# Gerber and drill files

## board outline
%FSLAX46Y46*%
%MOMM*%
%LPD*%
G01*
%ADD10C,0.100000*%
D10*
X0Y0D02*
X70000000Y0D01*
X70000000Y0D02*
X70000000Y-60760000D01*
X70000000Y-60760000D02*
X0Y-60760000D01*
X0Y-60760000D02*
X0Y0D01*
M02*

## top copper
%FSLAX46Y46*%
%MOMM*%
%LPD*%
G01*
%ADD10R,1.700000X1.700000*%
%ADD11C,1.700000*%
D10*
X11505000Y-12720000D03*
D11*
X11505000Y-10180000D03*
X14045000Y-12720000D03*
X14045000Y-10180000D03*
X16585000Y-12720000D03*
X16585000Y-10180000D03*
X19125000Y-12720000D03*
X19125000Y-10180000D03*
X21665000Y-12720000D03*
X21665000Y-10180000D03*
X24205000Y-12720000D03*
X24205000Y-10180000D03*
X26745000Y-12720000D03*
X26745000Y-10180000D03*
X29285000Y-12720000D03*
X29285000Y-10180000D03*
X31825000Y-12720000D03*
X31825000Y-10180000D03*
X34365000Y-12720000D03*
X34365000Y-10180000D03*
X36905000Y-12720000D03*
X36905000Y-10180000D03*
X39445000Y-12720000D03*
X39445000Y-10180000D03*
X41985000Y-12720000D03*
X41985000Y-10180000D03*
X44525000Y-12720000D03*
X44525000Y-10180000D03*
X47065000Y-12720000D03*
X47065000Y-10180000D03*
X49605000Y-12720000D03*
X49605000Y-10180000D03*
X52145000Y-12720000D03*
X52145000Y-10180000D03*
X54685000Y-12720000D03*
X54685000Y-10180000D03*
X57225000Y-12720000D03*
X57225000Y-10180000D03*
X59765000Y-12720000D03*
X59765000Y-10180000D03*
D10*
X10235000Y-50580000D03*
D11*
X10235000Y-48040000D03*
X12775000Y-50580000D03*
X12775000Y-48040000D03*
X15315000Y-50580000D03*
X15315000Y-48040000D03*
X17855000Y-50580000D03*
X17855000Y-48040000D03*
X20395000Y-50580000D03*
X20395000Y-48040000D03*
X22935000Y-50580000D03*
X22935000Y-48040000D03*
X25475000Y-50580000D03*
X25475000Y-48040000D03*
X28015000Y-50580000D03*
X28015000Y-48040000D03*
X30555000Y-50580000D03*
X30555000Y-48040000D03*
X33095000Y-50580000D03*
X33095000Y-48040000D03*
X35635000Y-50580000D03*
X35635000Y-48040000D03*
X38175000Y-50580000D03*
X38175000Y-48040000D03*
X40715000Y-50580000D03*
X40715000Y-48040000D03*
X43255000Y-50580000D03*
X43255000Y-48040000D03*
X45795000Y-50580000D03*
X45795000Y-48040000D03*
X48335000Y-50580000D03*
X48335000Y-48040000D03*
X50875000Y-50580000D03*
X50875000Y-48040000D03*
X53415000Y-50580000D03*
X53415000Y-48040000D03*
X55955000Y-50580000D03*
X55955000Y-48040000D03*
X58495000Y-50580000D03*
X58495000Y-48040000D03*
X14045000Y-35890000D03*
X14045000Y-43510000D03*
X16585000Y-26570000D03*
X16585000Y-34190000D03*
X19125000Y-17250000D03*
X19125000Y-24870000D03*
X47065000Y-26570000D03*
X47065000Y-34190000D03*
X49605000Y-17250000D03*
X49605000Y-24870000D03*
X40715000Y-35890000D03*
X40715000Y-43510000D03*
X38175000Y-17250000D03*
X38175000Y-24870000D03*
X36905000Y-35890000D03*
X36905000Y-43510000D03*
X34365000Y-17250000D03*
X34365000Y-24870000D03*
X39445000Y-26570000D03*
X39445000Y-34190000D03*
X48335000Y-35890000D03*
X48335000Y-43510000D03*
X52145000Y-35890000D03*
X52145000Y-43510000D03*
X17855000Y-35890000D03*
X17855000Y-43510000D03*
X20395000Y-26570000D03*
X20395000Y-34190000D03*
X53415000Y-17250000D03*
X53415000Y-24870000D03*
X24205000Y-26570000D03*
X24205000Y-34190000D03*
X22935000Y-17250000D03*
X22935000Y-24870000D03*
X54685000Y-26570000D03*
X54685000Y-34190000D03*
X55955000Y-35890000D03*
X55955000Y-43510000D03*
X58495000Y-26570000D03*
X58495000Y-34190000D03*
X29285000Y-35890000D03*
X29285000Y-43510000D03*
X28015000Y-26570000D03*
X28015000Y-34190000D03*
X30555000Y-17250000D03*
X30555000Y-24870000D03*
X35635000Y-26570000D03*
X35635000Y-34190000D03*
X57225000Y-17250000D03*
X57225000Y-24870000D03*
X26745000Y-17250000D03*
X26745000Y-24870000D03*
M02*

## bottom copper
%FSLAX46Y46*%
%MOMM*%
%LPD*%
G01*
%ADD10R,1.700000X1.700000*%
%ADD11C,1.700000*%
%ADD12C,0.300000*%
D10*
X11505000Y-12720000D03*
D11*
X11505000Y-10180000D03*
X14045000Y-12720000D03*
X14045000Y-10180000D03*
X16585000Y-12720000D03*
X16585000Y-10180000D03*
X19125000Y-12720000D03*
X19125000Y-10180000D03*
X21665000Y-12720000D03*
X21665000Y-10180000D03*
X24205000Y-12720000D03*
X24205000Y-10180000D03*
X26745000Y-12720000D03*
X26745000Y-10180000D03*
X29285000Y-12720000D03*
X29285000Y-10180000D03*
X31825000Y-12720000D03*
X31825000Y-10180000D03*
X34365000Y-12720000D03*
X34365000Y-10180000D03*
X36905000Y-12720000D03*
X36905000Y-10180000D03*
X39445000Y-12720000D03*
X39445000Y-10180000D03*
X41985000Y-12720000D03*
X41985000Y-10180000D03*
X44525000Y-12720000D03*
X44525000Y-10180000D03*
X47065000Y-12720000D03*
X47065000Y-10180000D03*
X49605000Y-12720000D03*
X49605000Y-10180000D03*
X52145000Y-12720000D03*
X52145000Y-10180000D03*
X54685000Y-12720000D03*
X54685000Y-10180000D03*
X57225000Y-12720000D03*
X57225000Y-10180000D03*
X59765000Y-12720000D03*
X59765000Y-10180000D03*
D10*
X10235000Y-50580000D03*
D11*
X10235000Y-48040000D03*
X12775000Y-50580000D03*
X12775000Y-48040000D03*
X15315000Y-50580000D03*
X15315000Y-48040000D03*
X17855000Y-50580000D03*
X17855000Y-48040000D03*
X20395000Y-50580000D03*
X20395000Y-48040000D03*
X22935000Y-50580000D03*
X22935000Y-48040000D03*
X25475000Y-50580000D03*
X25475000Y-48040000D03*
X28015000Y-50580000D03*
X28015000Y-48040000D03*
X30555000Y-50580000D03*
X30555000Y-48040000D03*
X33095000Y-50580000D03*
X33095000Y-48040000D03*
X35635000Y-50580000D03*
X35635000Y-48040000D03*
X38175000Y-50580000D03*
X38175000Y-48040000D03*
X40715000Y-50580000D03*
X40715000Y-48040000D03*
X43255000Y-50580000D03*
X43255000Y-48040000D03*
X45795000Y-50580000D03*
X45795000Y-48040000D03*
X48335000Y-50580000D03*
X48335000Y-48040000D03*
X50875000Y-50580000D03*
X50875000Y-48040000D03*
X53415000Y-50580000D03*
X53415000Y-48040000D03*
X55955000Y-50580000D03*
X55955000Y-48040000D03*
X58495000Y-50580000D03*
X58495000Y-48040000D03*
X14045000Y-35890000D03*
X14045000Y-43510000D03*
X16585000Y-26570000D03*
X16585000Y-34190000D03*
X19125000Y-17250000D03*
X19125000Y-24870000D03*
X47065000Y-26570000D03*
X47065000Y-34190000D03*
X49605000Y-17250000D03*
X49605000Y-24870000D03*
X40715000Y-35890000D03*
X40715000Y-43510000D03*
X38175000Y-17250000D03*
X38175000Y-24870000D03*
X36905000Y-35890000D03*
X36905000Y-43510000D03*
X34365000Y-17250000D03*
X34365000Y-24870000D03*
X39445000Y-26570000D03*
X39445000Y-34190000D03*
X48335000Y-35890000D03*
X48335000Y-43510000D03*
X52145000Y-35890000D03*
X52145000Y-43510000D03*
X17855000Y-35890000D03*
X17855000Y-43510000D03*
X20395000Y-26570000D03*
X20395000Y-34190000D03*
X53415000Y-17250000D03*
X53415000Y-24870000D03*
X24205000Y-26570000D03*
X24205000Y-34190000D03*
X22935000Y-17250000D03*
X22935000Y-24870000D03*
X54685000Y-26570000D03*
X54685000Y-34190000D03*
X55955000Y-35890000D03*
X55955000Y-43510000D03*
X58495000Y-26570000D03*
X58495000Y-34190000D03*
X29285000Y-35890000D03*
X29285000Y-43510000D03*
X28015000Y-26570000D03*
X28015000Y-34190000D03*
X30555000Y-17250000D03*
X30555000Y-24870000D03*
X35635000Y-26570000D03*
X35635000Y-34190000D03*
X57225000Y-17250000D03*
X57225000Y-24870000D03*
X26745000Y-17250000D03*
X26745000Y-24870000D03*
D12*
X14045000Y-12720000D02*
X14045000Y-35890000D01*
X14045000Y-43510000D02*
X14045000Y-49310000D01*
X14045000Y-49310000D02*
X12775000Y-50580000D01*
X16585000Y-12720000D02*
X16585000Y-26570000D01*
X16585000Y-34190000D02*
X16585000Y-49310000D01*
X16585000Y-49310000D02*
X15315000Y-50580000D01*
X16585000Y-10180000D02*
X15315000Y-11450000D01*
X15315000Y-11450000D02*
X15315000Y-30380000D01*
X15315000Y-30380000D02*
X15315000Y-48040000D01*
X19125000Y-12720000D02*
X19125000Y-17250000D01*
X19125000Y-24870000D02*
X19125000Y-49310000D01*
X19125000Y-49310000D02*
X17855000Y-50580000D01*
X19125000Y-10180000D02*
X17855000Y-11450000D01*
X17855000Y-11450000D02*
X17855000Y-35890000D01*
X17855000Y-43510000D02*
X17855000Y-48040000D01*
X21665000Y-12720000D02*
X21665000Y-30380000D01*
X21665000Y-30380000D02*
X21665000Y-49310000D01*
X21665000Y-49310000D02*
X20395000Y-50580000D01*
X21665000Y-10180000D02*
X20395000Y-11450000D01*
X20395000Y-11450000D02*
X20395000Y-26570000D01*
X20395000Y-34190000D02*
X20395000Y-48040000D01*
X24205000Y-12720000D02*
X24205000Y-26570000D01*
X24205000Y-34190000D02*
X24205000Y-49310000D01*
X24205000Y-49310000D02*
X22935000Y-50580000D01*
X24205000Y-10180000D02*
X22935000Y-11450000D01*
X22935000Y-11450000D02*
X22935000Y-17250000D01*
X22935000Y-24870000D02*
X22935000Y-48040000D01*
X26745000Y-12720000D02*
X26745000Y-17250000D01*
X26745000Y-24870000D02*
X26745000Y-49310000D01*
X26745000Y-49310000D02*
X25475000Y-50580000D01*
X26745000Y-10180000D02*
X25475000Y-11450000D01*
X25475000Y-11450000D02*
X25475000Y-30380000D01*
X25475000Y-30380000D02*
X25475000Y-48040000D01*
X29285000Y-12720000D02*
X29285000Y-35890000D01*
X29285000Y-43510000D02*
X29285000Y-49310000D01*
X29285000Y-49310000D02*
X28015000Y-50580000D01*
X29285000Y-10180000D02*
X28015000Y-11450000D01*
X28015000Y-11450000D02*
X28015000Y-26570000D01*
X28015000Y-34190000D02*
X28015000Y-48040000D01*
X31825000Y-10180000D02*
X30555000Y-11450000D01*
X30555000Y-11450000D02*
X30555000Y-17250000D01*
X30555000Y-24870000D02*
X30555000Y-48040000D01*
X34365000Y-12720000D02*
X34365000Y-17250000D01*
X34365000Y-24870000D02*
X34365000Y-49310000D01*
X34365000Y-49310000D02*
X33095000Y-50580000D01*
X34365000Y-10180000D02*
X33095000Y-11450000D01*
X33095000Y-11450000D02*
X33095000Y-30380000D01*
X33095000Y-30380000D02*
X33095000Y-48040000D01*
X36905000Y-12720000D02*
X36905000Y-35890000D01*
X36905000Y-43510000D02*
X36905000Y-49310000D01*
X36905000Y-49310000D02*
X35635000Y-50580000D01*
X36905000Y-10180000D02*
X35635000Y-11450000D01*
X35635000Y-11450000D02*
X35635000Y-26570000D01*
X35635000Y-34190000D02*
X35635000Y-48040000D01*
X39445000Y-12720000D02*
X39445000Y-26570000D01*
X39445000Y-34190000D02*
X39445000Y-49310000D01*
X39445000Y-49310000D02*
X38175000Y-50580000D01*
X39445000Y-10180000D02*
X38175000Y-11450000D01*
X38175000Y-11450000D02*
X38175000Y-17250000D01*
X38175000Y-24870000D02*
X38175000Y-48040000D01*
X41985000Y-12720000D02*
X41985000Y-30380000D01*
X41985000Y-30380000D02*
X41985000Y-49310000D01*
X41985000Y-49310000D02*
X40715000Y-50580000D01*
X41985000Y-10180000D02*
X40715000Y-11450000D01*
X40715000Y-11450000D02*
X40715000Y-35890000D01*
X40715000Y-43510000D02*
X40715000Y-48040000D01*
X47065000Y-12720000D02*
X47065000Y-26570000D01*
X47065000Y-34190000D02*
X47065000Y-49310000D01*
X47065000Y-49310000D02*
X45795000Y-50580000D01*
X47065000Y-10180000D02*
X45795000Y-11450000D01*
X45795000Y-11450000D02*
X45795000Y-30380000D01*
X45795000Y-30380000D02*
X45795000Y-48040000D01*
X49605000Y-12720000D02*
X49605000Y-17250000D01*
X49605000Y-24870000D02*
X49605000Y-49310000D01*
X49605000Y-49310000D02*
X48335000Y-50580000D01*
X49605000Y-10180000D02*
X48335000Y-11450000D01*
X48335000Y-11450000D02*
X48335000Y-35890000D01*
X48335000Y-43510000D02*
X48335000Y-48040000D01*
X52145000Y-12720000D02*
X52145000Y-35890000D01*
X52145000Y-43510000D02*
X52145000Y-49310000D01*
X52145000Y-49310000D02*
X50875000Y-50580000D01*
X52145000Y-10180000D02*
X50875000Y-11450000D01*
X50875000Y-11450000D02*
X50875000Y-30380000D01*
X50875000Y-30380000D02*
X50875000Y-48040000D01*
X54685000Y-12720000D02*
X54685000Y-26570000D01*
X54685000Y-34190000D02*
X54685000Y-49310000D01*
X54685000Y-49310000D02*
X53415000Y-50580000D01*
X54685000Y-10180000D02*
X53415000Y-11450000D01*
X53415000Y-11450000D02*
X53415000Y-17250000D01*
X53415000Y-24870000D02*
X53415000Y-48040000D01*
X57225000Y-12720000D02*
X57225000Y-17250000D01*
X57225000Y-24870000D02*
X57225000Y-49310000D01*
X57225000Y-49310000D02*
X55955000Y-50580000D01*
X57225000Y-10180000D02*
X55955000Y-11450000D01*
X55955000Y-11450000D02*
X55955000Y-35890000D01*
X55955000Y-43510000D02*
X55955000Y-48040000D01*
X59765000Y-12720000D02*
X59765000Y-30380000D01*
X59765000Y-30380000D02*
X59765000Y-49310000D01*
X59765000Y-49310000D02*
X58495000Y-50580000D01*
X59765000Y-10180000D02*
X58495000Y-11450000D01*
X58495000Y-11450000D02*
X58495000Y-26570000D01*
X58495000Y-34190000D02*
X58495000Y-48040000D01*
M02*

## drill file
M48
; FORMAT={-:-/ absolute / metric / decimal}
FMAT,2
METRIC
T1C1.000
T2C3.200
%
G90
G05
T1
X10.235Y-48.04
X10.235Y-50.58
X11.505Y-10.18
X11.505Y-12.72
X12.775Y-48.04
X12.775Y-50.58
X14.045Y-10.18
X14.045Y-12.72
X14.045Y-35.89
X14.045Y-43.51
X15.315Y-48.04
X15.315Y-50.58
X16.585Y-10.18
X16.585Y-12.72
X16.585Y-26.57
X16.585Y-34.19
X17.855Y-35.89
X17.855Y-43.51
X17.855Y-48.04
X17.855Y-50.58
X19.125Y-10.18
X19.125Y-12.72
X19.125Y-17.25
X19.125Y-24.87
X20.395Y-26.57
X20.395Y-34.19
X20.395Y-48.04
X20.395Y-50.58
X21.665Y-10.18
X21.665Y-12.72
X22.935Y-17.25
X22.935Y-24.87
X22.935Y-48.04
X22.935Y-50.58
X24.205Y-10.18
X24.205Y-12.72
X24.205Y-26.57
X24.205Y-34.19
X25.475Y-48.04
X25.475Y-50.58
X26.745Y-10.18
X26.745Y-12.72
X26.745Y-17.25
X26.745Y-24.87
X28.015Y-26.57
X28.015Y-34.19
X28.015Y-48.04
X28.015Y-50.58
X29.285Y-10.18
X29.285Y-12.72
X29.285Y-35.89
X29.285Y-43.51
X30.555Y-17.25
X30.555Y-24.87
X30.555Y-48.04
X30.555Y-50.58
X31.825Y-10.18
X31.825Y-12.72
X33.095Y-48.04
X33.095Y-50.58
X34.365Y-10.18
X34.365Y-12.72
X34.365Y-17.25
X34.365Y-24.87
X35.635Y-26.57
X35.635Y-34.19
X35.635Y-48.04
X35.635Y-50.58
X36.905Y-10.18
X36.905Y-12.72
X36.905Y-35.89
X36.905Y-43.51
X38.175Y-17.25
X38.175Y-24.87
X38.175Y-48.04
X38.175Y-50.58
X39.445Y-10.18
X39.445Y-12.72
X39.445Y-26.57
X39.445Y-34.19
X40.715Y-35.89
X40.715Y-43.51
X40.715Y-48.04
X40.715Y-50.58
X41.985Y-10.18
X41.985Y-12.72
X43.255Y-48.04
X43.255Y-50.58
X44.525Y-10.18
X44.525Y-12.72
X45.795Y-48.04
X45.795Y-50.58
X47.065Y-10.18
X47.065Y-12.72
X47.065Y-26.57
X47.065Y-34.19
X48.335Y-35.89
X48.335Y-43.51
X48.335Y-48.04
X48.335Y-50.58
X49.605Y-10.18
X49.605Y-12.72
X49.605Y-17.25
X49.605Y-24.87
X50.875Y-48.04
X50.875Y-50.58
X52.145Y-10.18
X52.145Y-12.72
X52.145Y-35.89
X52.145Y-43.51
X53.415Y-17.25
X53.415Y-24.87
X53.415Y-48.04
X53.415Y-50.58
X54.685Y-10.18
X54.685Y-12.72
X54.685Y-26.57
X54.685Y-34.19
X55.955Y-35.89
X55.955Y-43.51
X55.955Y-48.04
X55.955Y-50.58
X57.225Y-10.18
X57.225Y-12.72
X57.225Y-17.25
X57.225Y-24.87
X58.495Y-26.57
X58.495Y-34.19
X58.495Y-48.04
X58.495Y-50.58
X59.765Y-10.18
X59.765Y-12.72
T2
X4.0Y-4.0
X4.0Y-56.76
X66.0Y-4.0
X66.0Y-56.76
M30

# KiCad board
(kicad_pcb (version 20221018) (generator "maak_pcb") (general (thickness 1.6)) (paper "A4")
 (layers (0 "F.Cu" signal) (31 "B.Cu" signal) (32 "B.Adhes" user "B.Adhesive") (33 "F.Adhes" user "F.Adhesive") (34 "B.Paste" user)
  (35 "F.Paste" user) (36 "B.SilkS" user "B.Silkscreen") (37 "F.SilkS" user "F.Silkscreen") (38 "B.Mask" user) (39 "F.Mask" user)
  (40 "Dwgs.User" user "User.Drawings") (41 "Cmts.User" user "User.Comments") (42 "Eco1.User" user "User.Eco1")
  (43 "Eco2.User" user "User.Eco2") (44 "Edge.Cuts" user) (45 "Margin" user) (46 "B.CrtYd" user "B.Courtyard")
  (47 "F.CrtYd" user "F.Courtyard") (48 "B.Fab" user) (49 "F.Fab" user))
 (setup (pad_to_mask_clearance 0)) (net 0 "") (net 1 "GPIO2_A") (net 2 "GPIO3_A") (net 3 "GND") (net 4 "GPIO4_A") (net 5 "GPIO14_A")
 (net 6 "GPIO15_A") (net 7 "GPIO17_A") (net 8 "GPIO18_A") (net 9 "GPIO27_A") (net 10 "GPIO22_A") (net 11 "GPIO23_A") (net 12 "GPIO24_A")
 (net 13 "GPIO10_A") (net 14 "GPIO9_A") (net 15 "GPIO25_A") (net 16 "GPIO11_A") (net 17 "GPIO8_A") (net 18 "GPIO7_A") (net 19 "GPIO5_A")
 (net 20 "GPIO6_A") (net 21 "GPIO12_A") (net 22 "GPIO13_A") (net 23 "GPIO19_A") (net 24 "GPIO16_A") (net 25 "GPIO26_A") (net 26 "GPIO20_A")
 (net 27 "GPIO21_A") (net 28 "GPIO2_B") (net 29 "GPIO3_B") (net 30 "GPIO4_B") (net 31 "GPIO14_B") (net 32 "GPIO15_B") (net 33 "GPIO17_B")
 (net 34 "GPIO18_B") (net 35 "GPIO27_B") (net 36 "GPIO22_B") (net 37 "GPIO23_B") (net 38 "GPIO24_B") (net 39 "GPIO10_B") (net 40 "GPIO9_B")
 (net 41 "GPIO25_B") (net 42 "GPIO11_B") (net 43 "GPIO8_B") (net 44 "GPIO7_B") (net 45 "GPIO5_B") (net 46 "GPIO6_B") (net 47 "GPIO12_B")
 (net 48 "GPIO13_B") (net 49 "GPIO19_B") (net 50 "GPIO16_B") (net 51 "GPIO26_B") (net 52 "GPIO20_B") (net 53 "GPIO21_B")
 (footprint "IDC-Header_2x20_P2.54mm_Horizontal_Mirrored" (layer "F.Cu") (at 11.505 12.72)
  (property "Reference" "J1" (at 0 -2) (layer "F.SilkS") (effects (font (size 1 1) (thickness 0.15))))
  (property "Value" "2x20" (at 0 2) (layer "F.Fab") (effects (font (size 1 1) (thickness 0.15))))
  (pad "1" thru_hole rect (at 0 0) (size 1.7 1.7) (drill 1) (layers "B.Cu" "B.Mask"))
  (pad "2" thru_hole circle (at 0 -2.54) (size 1.7 1.7) (drill 1) (layers "B.Cu" "B.Mask"))
  (pad "3" thru_hole circle (at 2.54 0) (size 1.7 1.7) (drill 1) (layers "B.Cu" "B.Mask") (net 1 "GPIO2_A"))
  (pad "4" thru_hole circle (at 2.54 -2.54) (size 1.7 1.7) (drill 1) (layers "B.Cu" "B.Mask"))
  (pad "5" thru_hole circle (at 5.08 0) (size 1.7 1.7) (drill 1) (layers "B.Cu" "B.Mask") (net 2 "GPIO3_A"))
  (pad "6" thru_hole circle (at 5.08 -2.54) (size 1.7 1.7) (drill 1) (layers "B.Cu" "B.Mask") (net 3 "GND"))
  (pad "7" thru_hole circle (at 7.62 0) (size 1.7 1.7) (drill 1) (layers "B.Cu" "B.Mask") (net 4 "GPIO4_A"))
  (pad "8" thru_hole circle (at 7.62 -2.54) (size 1.7 1.7) (drill 1) (layers "B.Cu" "B.Mask") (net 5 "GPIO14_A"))
  (pad "9" thru_hole circle (at 10.16 0) (size 1.7 1.7) (drill 1) (layers "B.Cu" "B.Mask") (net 3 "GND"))
  (pad "10" thru_hole circle (at 10.16 -2.54) (size 1.7 1.7) (drill 1) (layers "B.Cu" "B.Mask") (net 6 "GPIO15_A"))
  (pad "11" thru_hole circle (at 12.7 0) (size 1.7 1.7) (drill 1) (layers "B.Cu" "B.Mask") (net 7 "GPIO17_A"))
  (pad "12" thru_hole circle (at 12.7 -2.54) (size 1.7 1.7) (drill 1) (layers "B.Cu" "B.Mask") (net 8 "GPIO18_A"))
  (pad "13" thru_hole circle (at 15.24 0) (size 1.7 1.7) (drill 1) (layers "B.Cu" "B.Mask") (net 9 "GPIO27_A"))
  (pad "14" thru_hole circle (at 15.24 -2.54) (size 1.7 1.7) (drill 1) (layers "B.Cu" "B.Mask") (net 3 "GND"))
  (pad "15" thru_hole circle (at 17.78 0) (size 1.7 1.7) (drill 1) (layers "B.Cu" "B.Mask") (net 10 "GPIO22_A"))
  (pad "16" thru_hole circle (at 17.78 -2.54) (size 1.7 1.7) (drill 1) (layers "B.Cu" "B.Mask") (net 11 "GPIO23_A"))
  (pad "17" thru_hole circle (at 20.32 0) (size 1.7 1.7) (drill 1) (layers "B.Cu" "B.Mask"))
  (pad "18" thru_hole circle (at 20.32 -2.54) (size 1.7 1.7) (drill 1) (layers "B.Cu" "B.Mask") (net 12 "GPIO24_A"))
  (pad "19" thru_hole circle (at 22.86 0) (size 1.7 1.7) (drill 1) (layers "B.Cu" "B.Mask") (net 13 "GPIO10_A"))
  (pad "20" thru_hole circle (at 22.86 -2.54) (size 1.7 1.7) (drill 1) (layers "B.Cu" "B.Mask") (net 3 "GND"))
  (pad "21" thru_hole circle (at 25.4 0) (size 1.7 1.7) (drill 1) (layers "B.Cu" "B.Mask") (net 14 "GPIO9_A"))
  (pad "22" thru_hole circle (at 25.4 -2.54) (size 1.7 1.7) (drill 1) (layers "B.Cu" "B.Mask") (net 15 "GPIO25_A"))
  (pad "23" thru_hole circle (at 27.94 0) (size 1.7 1.7) (drill 1) (layers "B.Cu" "B.Mask") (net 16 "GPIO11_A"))
  (pad "24" thru_hole circle (at 27.94 -2.54) (size 1.7 1.7) (drill 1) (layers "B.Cu" "B.Mask") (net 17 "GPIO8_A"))
  (pad "25" thru_hole circle (at 30.48 0) (size 1.7 1.7) (drill 1) (layers "B.Cu" "B.Mask") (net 3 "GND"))
  (pad "26" thru_hole circle (at 30.48 -2.54) (size 1.7 1.7) (drill 1) (layers "B.Cu" "B.Mask") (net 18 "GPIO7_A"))
  (pad "27" thru_hole circle (at 33.02 0) (size 1.7 1.7) (drill 1) (layers "B.Cu" "B.Mask"))
  (pad "28" thru_hole circle (at 33.02 -2.54) (size 1.7 1.7) (drill 1) (layers "B.Cu" "B.Mask"))
  (pad "29" thru_hole circle (at 35.56 0) (size 1.7 1.7) (drill 1) (layers "B.Cu" "B.Mask") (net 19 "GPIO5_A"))
  (pad "30" thru_hole circle (at 35.56 -2.54) (size 1.7 1.7) (drill 1) (layers "B.Cu" "B.Mask") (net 3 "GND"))
  (pad "31" thru_hole circle (at 38.1 0) (size 1.7 1.7) (drill 1) (layers "B.Cu" "B.Mask") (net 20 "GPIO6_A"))
  (pad "32" thru_hole circle (at 38.1 -2.54) (size 1.7 1.7) (drill 1) (layers "B.Cu" "B.Mask") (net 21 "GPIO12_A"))
  (pad "33" thru_hole circle (at 40.64 0) (size 1.7 1.7) (drill 1) (layers "B.Cu" "B.Mask") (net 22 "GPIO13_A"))
  (pad "34" thru_hole circle (at 40.64 -2.54) (size 1.7 1.7) (drill 1) (layers "B.Cu" "B.Mask") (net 3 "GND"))
  (pad "35" thru_hole circle (at 43.18 0) (size 1.7 1.7) (drill 1) (layers "B.Cu" "B.Mask") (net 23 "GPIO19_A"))
  (pad "36" thru_hole circle (at 43.18 -2.54) (size 1.7 1.7) (drill 1) (layers "B.Cu" "B.Mask") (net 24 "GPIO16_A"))
  (pad "37" thru_hole circle (at 45.72 0) (size 1.7 1.7) (drill 1) (layers "B.Cu" "B.Mask") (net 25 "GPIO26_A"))
  (pad "38" thru_hole circle (at 45.72 -2.54) (size 1.7 1.7) (drill 1) (layers "B.Cu" "B.Mask") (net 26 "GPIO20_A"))
  (pad "39" thru_hole circle (at 48.26 0) (size 1.7 1.7) (drill 1) (layers "B.Cu" "B.Mask") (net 3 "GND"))
  (pad "40" thru_hole circle (at 48.26 -2.54) (size 1.7 1.7) (drill 1) (layers "B.Cu" "B.Mask") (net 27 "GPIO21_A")))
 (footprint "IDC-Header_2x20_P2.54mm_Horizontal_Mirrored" (layer "F.Cu") (at 10.235 50.58)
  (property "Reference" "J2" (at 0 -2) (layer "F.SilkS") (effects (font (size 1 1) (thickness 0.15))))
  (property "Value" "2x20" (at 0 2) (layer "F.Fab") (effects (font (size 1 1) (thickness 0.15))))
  (pad "1" thru_hole rect (at 0 0) (size 1.7 1.7) (drill 1) (layers "B.Cu" "B.Mask"))
  (pad "2" thru_hole circle (at 0 -2.54) (size 1.7 1.7) (drill 1) (layers "B.Cu" "B.Mask"))
  (pad "3" thru_hole circle (at 2.54 0) (size 1.7 1.7) (drill 1) (layers "B.Cu" "B.Mask") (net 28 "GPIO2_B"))
  (pad "4" thru_hole circle (at 2.54 -2.54) (size 1.7 1.7) (drill 1) (layers "B.Cu" "B.Mask"))
  (pad "5" thru_hole circle (at 5.08 0) (size 1.7 1.7) (drill 1) (layers "B.Cu" "B.Mask") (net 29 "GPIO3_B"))
  (pad "6" thru_hole circle (at 5.08 -2.54) (size 1.7 1.7) (drill 1) (layers "B.Cu" "B.Mask") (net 3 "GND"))
  (pad "7" thru_hole circle (at 7.62 0) (size 1.7 1.7) (drill 1) (layers "B.Cu" "B.Mask") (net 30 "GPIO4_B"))
  (pad "8" thru_hole circle (at 7.62 -2.54) (size 1.7 1.7) (drill 1) (layers "B.Cu" "B.Mask") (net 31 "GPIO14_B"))
  (pad "9" thru_hole circle (at 10.16 0) (size 1.7 1.7) (drill 1) (layers "B.Cu" "B.Mask") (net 3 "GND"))
  (pad "10" thru_hole circle (at 10.16 -2.54) (size 1.7 1.7) (drill 1) (layers "B.Cu" "B.Mask") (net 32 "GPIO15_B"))
  (pad "11" thru_hole circle (at 12.7 0) (size 1.7 1.7) (drill 1) (layers "B.Cu" "B.Mask") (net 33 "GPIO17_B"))
  (pad "12" thru_hole circle (at 12.7 -2.54) (size 1.7 1.7) (drill 1) (layers "B.Cu" "B.Mask") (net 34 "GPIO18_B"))
  (pad "13" thru_hole circle (at 15.24 0) (size 1.7 1.7) (drill 1) (layers "B.Cu" "B.Mask") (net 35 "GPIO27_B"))
  (pad "14" thru_hole circle (at 15.24 -2.54) (size 1.7 1.7) (drill 1) (layers "B.Cu" "B.Mask") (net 3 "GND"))
  (pad "15" thru_hole circle (at 17.78 0) (size 1.7 1.7) (drill 1) (layers "B.Cu" "B.Mask") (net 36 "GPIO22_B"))
  (pad "16" thru_hole circle (at 17.78 -2.54) (size 1.7 1.7) (drill 1) (layers "B.Cu" "B.Mask") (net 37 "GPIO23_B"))
  (pad "17" thru_hole circle (at 20.32 0) (size 1.7 1.7) (drill 1) (layers "B.Cu" "B.Mask"))
  (pad "18" thru_hole circle (at 20.32 -2.54) (size 1.7 1.7) (drill 1) (layers "B.Cu" "B.Mask") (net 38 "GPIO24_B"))
  (pad "19" thru_hole circle (at 22.86 0) (size 1.7 1.7) (drill 1) (layers "B.Cu" "B.Mask") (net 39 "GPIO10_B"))
  (pad "20" thru_hole circle (at 22.86 -2.54) (size 1.7 1.7) (drill 1) (layers "B.Cu" "B.Mask") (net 3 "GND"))
  (pad "21" thru_hole circle (at 25.4 0) (size 1.7 1.7) (drill 1) (layers "B.Cu" "B.Mask") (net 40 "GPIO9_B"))
  (pad "22" thru_hole circle (at 25.4 -2.54) (size 1.7 1.7) (drill 1) (layers "B.Cu" "B.Mask") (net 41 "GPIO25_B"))
  (pad "23" thru_hole circle (at 27.94 0) (size 1.7 1.7) (drill 1) (layers "B.Cu" "B.Mask") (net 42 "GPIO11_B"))
  (pad "24" thru_hole circle (at 27.94 -2.54) (size 1.7 1.7) (drill 1) (layers "B.Cu" "B.Mask") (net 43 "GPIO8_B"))
  (pad "25" thru_hole circle (at 30.48 0) (size 1.7 1.7) (drill 1) (layers "B.Cu" "B.Mask") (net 3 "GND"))
  (pad "26" thru_hole circle (at 30.48 -2.54) (size 1.7 1.7) (drill 1) (layers "B.Cu" "B.Mask") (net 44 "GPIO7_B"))
  (pad "27" thru_hole circle (at 33.02 0) (size 1.7 1.7) (drill 1) (layers "B.Cu" "B.Mask"))
  (pad "28" thru_hole circle (at 33.02 -2.54) (size 1.7 1.7) (drill 1) (layers "B.Cu" "B.Mask"))
  (pad "29" thru_hole circle (at 35.56 0) (size 1.7 1.7) (drill 1) (layers "B.Cu" "B.Mask") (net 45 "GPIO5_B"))
  (pad "30" thru_hole circle (at 35.56 -2.54) (size 1.7 1.7) (drill 1) (layers "B.Cu" "B.Mask") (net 3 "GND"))
  (pad "31" thru_hole circle (at 38.1 0) (size 1.7 1.7) (drill 1) (layers "B.Cu" "B.Mask") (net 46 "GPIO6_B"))
  (pad "32" thru_hole circle (at 38.1 -2.54) (size 1.7 1.7) (drill 1) (layers "B.Cu" "B.Mask") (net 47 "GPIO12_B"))
  (pad "33" thru_hole circle (at 40.64 0) (size 1.7 1.7) (drill 1) (layers "B.Cu" "B.Mask") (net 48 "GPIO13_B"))
  (pad "34" thru_hole circle (at 40.64 -2.54) (size 1.7 1.7) (drill 1) (layers "B.Cu" "B.Mask") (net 3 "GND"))
  (pad "35" thru_hole circle (at 43.18 0) (size 1.7 1.7) (drill 1) (layers "B.Cu" "B.Mask") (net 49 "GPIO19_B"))
  (pad "36" thru_hole circle (at 43.18 -2.54) (size 1.7 1.7) (drill 1) (layers "B.Cu" "B.Mask") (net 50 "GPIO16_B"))
  (pad "37" thru_hole circle (at 45.72 0) (size 1.7 1.7) (drill 1) (layers "B.Cu" "B.Mask") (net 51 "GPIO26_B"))
  (pad "38" thru_hole circle (at 45.72 -2.54) (size 1.7 1.7) (drill 1) (layers "B.Cu" "B.Mask") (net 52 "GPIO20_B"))
  (pad "39" thru_hole circle (at 48.26 0) (size 1.7 1.7) (drill 1) (layers "B.Cu" "B.Mask") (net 3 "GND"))
  (pad "40" thru_hole circle (at 48.26 -2.54) (size 1.7 1.7) (drill 1) (layers "B.Cu" "B.Mask") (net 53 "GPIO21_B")))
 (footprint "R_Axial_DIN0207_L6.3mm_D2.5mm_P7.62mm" (layer "F.Cu") (at 14.045 35.89)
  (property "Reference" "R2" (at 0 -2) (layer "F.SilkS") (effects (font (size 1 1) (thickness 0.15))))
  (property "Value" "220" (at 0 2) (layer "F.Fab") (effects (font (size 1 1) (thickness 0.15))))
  (pad "1" thru_hole circle (at 0 0) (size 1.7 1.7) (drill 1) (layers "B.Cu" "B.Mask") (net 1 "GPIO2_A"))
  (pad "2" thru_hole circle (at 0 7.62) (size 1.7 1.7) (drill 1) (layers "B.Cu" "B.Mask") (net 28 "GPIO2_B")))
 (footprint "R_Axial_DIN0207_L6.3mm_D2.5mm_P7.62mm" (layer "F.Cu") (at 16.585 26.57)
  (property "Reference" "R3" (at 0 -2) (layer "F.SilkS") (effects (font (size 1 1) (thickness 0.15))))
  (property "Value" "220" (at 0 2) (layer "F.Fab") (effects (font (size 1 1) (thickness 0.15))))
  (pad "1" thru_hole circle (at 0 0) (size 1.7 1.7) (drill 1) (layers "B.Cu" "B.Mask") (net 2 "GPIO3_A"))
  (pad "2" thru_hole circle (at 0 7.62) (size 1.7 1.7) (drill 1) (layers "B.Cu" "B.Mask") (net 29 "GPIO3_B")))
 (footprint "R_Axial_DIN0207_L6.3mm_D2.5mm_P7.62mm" (layer "F.Cu") (at 19.125 17.25)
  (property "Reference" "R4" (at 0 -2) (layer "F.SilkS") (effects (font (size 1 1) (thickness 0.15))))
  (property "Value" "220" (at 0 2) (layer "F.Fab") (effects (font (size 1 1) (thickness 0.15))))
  (pad "1" thru_hole circle (at 0 0) (size 1.7 1.7) (drill 1) (layers "B.Cu" "B.Mask") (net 4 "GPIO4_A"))
  (pad "2" thru_hole circle (at 0 7.62) (size 1.7 1.7) (drill 1) (layers "B.Cu" "B.Mask") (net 30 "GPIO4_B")))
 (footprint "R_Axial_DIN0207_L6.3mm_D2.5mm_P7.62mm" (layer "F.Cu") (at 47.065 26.57)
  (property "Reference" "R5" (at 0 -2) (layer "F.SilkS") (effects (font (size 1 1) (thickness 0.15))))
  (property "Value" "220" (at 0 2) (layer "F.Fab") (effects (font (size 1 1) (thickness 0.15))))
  (pad "1" thru_hole circle (at 0 0) (size 1.7 1.7) (drill 1) (layers "B.Cu" "B.Mask") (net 19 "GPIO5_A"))
  (pad "2" thru_hole circle (at 0 7.62) (size 1.7 1.7) (drill 1) (layers "B.Cu" "B.Mask") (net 45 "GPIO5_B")))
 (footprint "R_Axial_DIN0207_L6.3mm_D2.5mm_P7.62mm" (layer "F.Cu") (at 49.605 17.25)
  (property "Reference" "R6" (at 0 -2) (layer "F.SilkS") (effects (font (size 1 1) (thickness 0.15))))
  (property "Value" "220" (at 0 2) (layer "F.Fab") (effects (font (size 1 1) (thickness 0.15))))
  (pad "1" thru_hole circle (at 0 0) (size 1.7 1.7) (drill 1) (layers "B.Cu" "B.Mask") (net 20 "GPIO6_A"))
  (pad "2" thru_hole circle (at 0 7.62) (size 1.7 1.7) (drill 1) (layers "B.Cu" "B.Mask") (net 46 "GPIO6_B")))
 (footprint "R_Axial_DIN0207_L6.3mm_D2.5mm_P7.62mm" (layer "F.Cu") (at 40.715 35.89)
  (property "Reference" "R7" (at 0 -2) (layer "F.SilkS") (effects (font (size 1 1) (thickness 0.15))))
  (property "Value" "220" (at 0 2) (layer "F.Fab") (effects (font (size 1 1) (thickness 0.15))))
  (pad "1" thru_hole circle (at 0 0) (size 1.7 1.7) (drill 1) (layers "B.Cu" "B.Mask") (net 18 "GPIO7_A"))
  (pad "2" thru_hole circle (at 0 7.62) (size 1.7 1.7) (drill 1) (layers "B.Cu" "B.Mask") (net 44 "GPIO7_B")))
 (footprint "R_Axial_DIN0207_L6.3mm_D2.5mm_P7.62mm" (layer "F.Cu") (at 38.175 17.25)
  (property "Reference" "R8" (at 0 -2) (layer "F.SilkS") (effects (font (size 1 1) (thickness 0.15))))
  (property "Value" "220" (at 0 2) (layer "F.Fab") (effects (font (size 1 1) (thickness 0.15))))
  (pad "1" thru_hole circle (at 0 0) (size 1.7 1.7) (drill 1) (layers "B.Cu" "B.Mask") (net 17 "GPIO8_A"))
  (pad "2" thru_hole circle (at 0 7.62) (size 1.7 1.7) (drill 1) (layers "B.Cu" "B.Mask") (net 43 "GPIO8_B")))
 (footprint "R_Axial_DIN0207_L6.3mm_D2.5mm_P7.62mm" (layer "F.Cu") (at 36.905 35.89)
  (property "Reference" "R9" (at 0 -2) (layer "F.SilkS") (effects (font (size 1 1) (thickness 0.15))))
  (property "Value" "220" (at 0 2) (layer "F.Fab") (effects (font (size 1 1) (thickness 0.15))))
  (pad "1" thru_hole circle (at 0 0) (size 1.7 1.7) (drill 1) (layers "B.Cu" "B.Mask") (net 14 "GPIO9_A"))
  (pad "2" thru_hole circle (at 0 7.62) (size 1.7 1.7) (drill 1) (layers "B.Cu" "B.Mask") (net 40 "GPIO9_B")))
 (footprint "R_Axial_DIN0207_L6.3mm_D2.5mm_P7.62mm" (layer "F.Cu") (at 34.365 17.25)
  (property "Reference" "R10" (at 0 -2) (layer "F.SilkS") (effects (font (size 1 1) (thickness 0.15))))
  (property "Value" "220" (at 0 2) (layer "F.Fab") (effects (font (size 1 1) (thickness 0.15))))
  (pad "1" thru_hole circle (at 0 0) (size 1.7 1.7) (drill 1) (layers "B.Cu" "B.Mask") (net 13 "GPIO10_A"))
  (pad "2" thru_hole circle (at 0 7.62) (size 1.7 1.7) (drill 1) (layers "B.Cu" "B.Mask") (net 39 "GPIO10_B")))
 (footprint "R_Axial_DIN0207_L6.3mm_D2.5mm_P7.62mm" (layer "F.Cu") (at 39.445 26.57)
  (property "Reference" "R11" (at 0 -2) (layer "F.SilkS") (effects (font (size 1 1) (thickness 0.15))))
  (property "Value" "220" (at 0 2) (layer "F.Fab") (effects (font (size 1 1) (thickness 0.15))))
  (pad "1" thru_hole circle (at 0 0) (size 1.7 1.7) (drill 1) (layers "B.Cu" "B.Mask") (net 16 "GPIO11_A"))
  (pad "2" thru_hole circle (at 0 7.62) (size 1.7 1.7) (drill 1) (layers "B.Cu" "B.Mask") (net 42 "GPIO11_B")))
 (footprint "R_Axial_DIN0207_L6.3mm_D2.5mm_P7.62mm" (layer "F.Cu") (at 48.335 35.89)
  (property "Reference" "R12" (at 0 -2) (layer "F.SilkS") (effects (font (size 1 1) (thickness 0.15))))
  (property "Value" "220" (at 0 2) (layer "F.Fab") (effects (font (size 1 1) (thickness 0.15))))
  (pad "1" thru_hole circle (at 0 0) (size 1.7 1.7) (drill 1) (layers "B.Cu" "B.Mask") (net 21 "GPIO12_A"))
  (pad "2" thru_hole circle (at 0 7.62) (size 1.7 1.7) (drill 1) (layers "B.Cu" "B.Mask") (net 47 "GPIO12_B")))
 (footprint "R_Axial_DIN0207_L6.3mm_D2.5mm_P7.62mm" (layer "F.Cu") (at 52.145 35.89)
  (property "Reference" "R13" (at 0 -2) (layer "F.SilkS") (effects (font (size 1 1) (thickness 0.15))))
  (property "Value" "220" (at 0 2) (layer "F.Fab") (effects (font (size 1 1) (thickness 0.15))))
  (pad "1" thru_hole circle (at 0 0) (size 1.7 1.7) (drill 1) (layers "B.Cu" "B.Mask") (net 22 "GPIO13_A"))
  (pad "2" thru_hole circle (at 0 7.62) (size 1.7 1.7) (drill 1) (layers "B.Cu" "B.Mask") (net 48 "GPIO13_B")))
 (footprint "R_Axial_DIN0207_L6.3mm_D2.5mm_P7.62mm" (layer "F.Cu") (at 17.855 35.89)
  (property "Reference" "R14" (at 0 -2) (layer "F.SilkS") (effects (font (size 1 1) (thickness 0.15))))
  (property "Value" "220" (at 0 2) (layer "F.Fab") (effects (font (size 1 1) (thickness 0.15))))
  (pad "1" thru_hole circle (at 0 0) (size 1.7 1.7) (drill 1) (layers "B.Cu" "B.Mask") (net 5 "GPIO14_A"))
  (pad "2" thru_hole circle (at 0 7.62) (size 1.7 1.7) (drill 1) (layers "B.Cu" "B.Mask") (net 31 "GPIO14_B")))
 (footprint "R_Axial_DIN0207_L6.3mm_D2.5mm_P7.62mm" (layer "F.Cu") (at 20.395 26.57)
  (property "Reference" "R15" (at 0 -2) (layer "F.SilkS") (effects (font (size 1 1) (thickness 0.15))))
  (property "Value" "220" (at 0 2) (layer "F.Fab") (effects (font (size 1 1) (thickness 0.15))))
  (pad "1" thru_hole circle (at 0 0) (size 1.7 1.7) (drill 1) (layers "B.Cu" "B.Mask") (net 6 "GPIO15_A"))
  (pad "2" thru_hole circle (at 0 7.62) (size 1.7 1.7) (drill 1) (layers "B.Cu" "B.Mask") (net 32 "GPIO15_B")))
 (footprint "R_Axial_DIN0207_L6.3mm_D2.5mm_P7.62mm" (layer "F.Cu") (at 53.415 17.25)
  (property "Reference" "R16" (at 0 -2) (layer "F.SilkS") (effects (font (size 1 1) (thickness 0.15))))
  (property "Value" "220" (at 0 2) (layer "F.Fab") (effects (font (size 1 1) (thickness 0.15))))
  (pad "1" thru_hole circle (at 0 0) (size 1.7 1.7) (drill 1) (layers "B.Cu" "B.Mask") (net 24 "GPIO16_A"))
  (pad "2" thru_hole circle (at 0 7.62) (size 1.7 1.7) (drill 1) (layers "B.Cu" "B.Mask") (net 50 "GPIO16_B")))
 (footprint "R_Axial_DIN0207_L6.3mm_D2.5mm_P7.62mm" (layer "F.Cu") (at 24.205 26.57)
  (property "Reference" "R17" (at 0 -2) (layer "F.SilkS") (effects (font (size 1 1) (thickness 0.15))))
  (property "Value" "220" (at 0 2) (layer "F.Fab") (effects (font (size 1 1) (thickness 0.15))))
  (pad "1" thru_hole circle (at 0 0) (size 1.7 1.7) (drill 1) (layers "B.Cu" "B.Mask") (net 7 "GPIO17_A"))
  (pad "2" thru_hole circle (at 0 7.62) (size 1.7 1.7) (drill 1) (layers "B.Cu" "B.Mask") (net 33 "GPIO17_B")))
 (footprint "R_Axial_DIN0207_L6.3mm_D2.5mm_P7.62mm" (layer "F.Cu") (at 22.935 17.25)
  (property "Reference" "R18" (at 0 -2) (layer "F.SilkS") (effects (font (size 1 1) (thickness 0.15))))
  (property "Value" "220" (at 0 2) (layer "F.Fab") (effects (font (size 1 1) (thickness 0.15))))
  (pad "1" thru_hole circle (at 0 0) (size 1.7 1.7) (drill 1) (layers "B.Cu" "B.Mask") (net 8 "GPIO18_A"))
  (pad "2" thru_hole circle (at 0 7.62) (size 1.7 1.7) (drill 1) (layers "B.Cu" "B.Mask") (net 34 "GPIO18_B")))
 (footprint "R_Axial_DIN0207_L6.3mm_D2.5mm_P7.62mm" (layer "F.Cu") (at 54.685 26.57)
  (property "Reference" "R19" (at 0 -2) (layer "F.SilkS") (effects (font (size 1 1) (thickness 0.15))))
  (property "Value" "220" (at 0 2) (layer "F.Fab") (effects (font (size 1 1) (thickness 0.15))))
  (pad "1" thru_hole circle (at 0 0) (size 1.7 1.7) (drill 1) (layers "B.Cu" "B.Mask") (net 23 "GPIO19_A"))
  (pad "2" thru_hole circle (at 0 7.62) (size 1.7 1.7) (drill 1) (layers "B.Cu" "B.Mask") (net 49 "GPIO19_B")))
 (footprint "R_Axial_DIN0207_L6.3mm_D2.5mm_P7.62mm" (layer "F.Cu") (at 55.955 35.89)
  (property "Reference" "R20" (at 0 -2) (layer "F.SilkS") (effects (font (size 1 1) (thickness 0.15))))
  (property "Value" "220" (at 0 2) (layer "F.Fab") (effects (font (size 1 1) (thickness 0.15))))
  (pad "1" thru_hole circle (at 0 0) (size 1.7 1.7) (drill 1) (layers "B.Cu" "B.Mask") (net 26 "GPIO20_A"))
  (pad "2" thru_hole circle (at 0 7.62) (size 1.7 1.7) (drill 1) (layers "B.Cu" "B.Mask") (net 52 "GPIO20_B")))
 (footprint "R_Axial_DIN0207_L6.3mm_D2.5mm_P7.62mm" (layer "F.Cu") (at 58.495 26.57)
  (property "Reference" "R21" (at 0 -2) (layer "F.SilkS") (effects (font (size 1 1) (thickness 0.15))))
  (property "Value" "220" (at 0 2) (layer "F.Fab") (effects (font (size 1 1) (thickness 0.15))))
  (pad "1" thru_hole circle (at 0 0) (size 1.7 1.7) (drill 1) (layers "B.Cu" "B.Mask") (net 27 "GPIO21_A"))
  (pad "2" thru_hole circle (at 0 7.62) (size 1.7 1.7) (drill 1) (layers "B.Cu" "B.Mask") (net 53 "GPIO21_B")))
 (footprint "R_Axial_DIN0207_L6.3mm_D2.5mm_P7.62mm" (layer "F.Cu") (at 29.285 35.89)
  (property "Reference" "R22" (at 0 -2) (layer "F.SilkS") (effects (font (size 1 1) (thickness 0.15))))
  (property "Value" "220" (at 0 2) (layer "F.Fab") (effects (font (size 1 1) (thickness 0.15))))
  (pad "1" thru_hole circle (at 0 0) (size 1.7 1.7) (drill 1) (layers "B.Cu" "B.Mask") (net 10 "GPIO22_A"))
  (pad "2" thru_hole circle (at 0 7.62) (size 1.7 1.7) (drill 1) (layers "B.Cu" "B.Mask") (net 36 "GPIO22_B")))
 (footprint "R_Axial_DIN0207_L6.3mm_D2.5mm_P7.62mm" (layer "F.Cu") (at 28.015 26.57)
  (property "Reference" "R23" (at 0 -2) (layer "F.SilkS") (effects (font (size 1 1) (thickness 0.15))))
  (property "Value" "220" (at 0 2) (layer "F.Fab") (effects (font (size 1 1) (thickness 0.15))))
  (pad "1" thru_hole circle (at 0 0) (size 1.7 1.7) (drill 1) (layers "B.Cu" "B.Mask") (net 11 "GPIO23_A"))
  (pad "2" thru_hole circle (at 0 7.62) (size 1.7 1.7) (drill 1) (layers "B.Cu" "B.Mask") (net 37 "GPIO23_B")))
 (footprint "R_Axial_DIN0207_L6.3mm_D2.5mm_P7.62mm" (layer "F.Cu") (at 30.555 17.25)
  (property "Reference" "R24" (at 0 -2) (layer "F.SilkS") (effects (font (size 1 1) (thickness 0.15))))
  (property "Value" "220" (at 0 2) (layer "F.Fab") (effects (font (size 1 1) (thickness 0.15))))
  (pad "1" thru_hole circle (at 0 0) (size 1.7 1.7) (drill 1) (layers "B.Cu" "B.Mask") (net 12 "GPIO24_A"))
  (pad "2" thru_hole circle (at 0 7.62) (size 1.7 1.7) (drill 1) (layers "B.Cu" "B.Mask") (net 38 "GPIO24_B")))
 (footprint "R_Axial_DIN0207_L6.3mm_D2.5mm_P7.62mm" (layer "F.Cu") (at 35.635 26.57)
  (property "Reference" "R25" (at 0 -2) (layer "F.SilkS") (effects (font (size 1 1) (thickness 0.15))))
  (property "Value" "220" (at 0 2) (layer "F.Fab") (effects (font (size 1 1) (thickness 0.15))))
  (pad "1" thru_hole circle (at 0 0) (size 1.7 1.7) (drill 1) (layers "B.Cu" "B.Mask") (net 15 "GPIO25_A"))
  (pad "2" thru_hole circle (at 0 7.62) (size 1.7 1.7) (drill 1) (layers "B.Cu" "B.Mask") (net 41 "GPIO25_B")))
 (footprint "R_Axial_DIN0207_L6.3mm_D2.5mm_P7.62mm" (layer "F.Cu") (at 57.225 17.25)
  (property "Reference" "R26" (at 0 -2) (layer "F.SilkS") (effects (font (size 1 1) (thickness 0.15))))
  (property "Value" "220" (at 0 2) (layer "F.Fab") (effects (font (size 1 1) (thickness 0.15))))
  (pad "1" thru_hole circle (at 0 0) (size 1.7 1.7) (drill 1) (layers "B.Cu" "B.Mask") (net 25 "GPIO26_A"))
  (pad "2" thru_hole circle (at 0 7.62) (size 1.7 1.7) (drill 1) (layers "B.Cu" "B.Mask") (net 51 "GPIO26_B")))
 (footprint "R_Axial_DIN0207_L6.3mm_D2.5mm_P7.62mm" (layer "F.Cu") (at 26.745 17.25)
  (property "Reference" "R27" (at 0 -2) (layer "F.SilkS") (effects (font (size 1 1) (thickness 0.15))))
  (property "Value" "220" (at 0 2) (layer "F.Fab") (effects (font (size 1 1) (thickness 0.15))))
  (pad "1" thru_hole circle (at 0 0) (size 1.7 1.7) (drill 1) (layers "B.Cu" "B.Mask") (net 9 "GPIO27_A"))
  (pad "2" thru_hole circle (at 0 7.62) (size 1.7 1.7) (drill 1) (layers "B.Cu" "B.Mask") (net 35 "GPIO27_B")))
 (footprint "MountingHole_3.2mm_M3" (layer "F.Cu") (at 4 4)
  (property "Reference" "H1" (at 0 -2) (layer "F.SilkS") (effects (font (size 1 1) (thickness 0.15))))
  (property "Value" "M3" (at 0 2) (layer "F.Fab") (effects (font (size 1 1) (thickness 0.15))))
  (pad "" np_thru_hole circle (at 0 0) (size 3.2 3.2) (drill 3.2) (layers "*.Cu" "*.Mask")))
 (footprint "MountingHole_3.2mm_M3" (layer "F.Cu") (at 66 4)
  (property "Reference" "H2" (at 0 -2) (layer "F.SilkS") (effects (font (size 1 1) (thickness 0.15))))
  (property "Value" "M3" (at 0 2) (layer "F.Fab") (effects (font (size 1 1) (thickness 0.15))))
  (pad "" np_thru_hole circle (at 0 0) (size 3.2 3.2) (drill 3.2) (layers "*.Cu" "*.Mask")))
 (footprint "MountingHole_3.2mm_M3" (layer "F.Cu") (at 4 56.76)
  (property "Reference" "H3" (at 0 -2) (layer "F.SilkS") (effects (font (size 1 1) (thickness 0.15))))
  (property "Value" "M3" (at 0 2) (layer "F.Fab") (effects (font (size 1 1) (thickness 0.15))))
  (pad "" np_thru_hole circle (at 0 0) (size 3.2 3.2) (drill 3.2) (layers "*.Cu" "*.Mask")))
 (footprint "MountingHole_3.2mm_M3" (layer "F.Cu") (at 66 56.76)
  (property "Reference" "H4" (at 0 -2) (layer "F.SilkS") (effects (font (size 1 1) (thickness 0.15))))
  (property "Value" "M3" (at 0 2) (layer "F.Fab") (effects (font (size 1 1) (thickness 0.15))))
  (pad "" np_thru_hole circle (at 0 0) (size 3.2 3.2) (drill 3.2) (layers "*.Cu" "*.Mask")))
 (segment (start 14.045 12.72) (end 14.045 35.89) (width 0.3) (layer "B.Cu") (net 1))
 (segment (start 14.045 43.51) (end 14.045 49.31) (width 0.3) (layer "B.Cu") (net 28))
 (segment (start 14.045 49.31) (end 12.775 50.58) (width 0.3) (layer "B.Cu") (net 28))
 (segment (start 16.585 12.72) (end 16.585 26.57) (width 0.3) (layer "B.Cu") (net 2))
 (segment (start 16.585 34.19) (end 16.585 49.31) (width 0.3) (layer "B.Cu") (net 29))
 (segment (start 16.585 49.31) (end 15.315 50.58) (width 0.3) (layer "B.Cu") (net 29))
 (segment (start 16.585 10.18) (end 15.315 11.45) (width 0.3) (layer "B.Cu") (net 3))
 (segment (start 15.315 11.45) (end 15.315 30.38) (width 0.3) (layer "B.Cu") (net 3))
 (segment (start 15.315 30.38) (end 15.315 48.04) (width 0.3) (layer "B.Cu") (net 3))
 (segment (start 19.125 12.72) (end 19.125 17.25) (width 0.3) (layer "B.Cu") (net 4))
 (segment (start 19.125 24.87) (end 19.125 49.31) (width 0.3) (layer "B.Cu") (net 30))
 (segment (start 19.125 49.31) (end 17.855 50.58) (width 0.3) (layer "B.Cu") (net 30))
 (segment (start 19.125 10.18) (end 17.855 11.45) (width 0.3) (layer "B.Cu") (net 5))
 (segment (start 17.855 11.45) (end 17.855 35.89) (width 0.3) (layer "B.Cu") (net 5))
 (segment (start 17.855 43.51) (end 17.855 48.04) (width 0.3) (layer "B.Cu") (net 31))
 (segment (start 21.665 12.72) (end 21.665 30.38) (width 0.3) (layer "B.Cu") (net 3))
 (segment (start 21.665 30.38) (end 21.665 49.31) (width 0.3) (layer "B.Cu") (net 3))
 (segment (start 21.665 49.31) (end 20.395 50.58) (width 0.3) (layer "B.Cu") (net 3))
 (segment (start 21.665 10.18) (end 20.395 11.45) (width 0.3) (layer "B.Cu") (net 6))
 (segment (start 20.395 11.45) (end 20.395 26.57) (width 0.3) (layer "B.Cu") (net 6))
 (segment (start 20.395 34.19) (end 20.395 48.04) (width 0.3) (layer "B.Cu") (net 32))
 (segment (start 24.205 12.72) (end 24.205 26.57) (width 0.3) (layer "B.Cu") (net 7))
 (segment (start 24.205 34.19) (end 24.205 49.31) (width 0.3) (layer "B.Cu") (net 33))
 (segment (start 24.205 49.31) (end 22.935 50.58) (width 0.3) (layer "B.Cu") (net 33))
 (segment (start 24.205 10.18) (end 22.935 11.45) (width 0.3) (layer "B.Cu") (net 8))
 (segment (start 22.935 11.45) (end 22.935 17.25) (width 0.3) (layer "B.Cu") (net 8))
 (segment (start 22.935 24.87) (end 22.935 48.04) (width 0.3) (layer "B.Cu") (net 34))
 (segment (start 26.745 12.72) (end 26.745 17.25) (width 0.3) (layer "B.Cu") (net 9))
 (segment (start 26.745 24.87) (end 26.745 49.31) (width 0.3) (layer "B.Cu") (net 35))
 (segment (start 26.745 49.31) (end 25.475 50.58) (width 0.3) (layer "B.Cu") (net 35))
 (segment (start 26.745 10.18) (end 25.475 11.45) (width 0.3) (layer "B.Cu") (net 3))
 (segment (start 25.475 11.45) (end 25.475 30.38) (width 0.3) (layer "B.Cu") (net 3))
 (segment (start 25.475 30.38) (end 25.475 48.04) (width 0.3) (layer "B.Cu") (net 3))
 (segment (start 29.285 12.72) (end 29.285 35.89) (width 0.3) (layer "B.Cu") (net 10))
 (segment (start 29.285 43.51) (end 29.285 49.31) (width 0.3) (layer "B.Cu") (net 36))
 (segment (start 29.285 49.31) (end 28.015 50.58) (width 0.3) (layer "B.Cu") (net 36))
 (segment (start 29.285 10.18) (end 28.015 11.45) (width 0.3) (layer "B.Cu") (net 11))
 (segment (start 28.015 11.45) (end 28.015 26.57) (width 0.3) (layer "B.Cu") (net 11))
 (segment (start 28.015 34.19) (end 28.015 48.04) (width 0.3) (layer "B.Cu") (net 37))
 (segment (start 31.825 10.18) (end 30.555 11.45) (width 0.3) (layer "B.Cu") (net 12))
 (segment (start 30.555 11.45) (end 30.555 17.25) (width 0.3) (layer "B.Cu") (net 12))
 (segment (start 30.555 24.87) (end 30.555 48.04) (width 0.3) (layer "B.Cu") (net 38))
 (segment (start 34.365 12.72) (end 34.365 17.25) (width 0.3) (layer "B.Cu") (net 13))
 (segment (start 34.365 24.87) (end 34.365 49.31) (width 0.3) (layer "B.Cu") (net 39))
 (segment (start 34.365 49.31) (end 33.095 50.58) (width 0.3) (layer "B.Cu") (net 39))
 (segment (start 34.365 10.18) (end 33.095 11.45) (width 0.3) (layer "B.Cu") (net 3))
 (segment (start 33.095 11.45) (end 33.095 30.38) (width 0.3) (layer "B.Cu") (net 3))
 (segment (start 33.095 30.38) (end 33.095 48.04) (width 0.3) (layer "B.Cu") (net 3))
 (segment (start 36.905 12.72) (end 36.905 35.89) (width 0.3) (layer "B.Cu") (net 14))
 (segment (start 36.905 43.51) (end 36.905 49.31) (width 0.3) (layer "B.Cu") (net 40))
 (segment (start 36.905 49.31) (end 35.635 50.58) (width 0.3) (layer "B.Cu") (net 40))
 (segment (start 36.905 10.18) (end 35.635 11.45) (width 0.3) (layer "B.Cu") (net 15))
 (segment (start 35.635 11.45) (end 35.635 26.57) (width 0.3) (layer "B.Cu") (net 15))
 (segment (start 35.635 34.19) (end 35.635 48.04) (width 0.3) (layer "B.Cu") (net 41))
 (segment (start 39.445 12.72) (end 39.445 26.57) (width 0.3) (layer "B.Cu") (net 16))
 (segment (start 39.445 34.19) (end 39.445 49.31) (width 0.3) (layer "B.Cu") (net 42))
 (segment (start 39.445 49.31) (end 38.175 50.58) (width 0.3) (layer "B.Cu") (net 42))
 (segment (start 39.445 10.18) (end 38.175 11.45) (width 0.3) (layer "B.Cu") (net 17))
 (segment (start 38.175 11.45) (end 38.175 17.25) (width 0.3) (layer "B.Cu") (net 17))
 (segment (start 38.175 24.87) (end 38.175 48.04) (width 0.3) (layer "B.Cu") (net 43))
 (segment (start 41.985 12.72) (end 41.985 30.38) (width 0.3) (layer "B.Cu") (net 3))
 (segment (start 41.985 30.38) (end 41.985 49.31) (width 0.3) (layer "B.Cu") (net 3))
 (segment (start 41.985 49.31) (end 40.715 50.58) (width 0.3) (layer "B.Cu") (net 3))
 (segment (start 41.985 10.18) (end 40.715 11.45) (width 0.3) (layer "B.Cu") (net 18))
 (segment (start 40.715 11.45) (end 40.715 35.89) (width 0.3) (layer "B.Cu") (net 18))
 (segment (start 40.715 43.51) (end 40.715 48.04) (width 0.3) (layer "B.Cu") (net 44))
 (segment (start 47.065 12.72) (end 47.065 26.57) (width 0.3) (layer "B.Cu") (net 19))
 (segment (start 47.065 34.19) (end 47.065 49.31) (width 0.3) (layer "B.Cu") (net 45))
 (segment (start 47.065 49.31) (end 45.795 50.58) (width 0.3) (layer "B.Cu") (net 45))
 (segment (start 47.065 10.18) (end 45.795 11.45) (width 0.3) (layer "B.Cu") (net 3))
 (segment (start 45.795 11.45) (end 45.795 30.38) (width 0.3) (layer "B.Cu") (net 3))
 (segment (start 45.795 30.38) (end 45.795 48.04) (width 0.3) (layer "B.Cu") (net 3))
 (segment (start 49.605 12.72) (end 49.605 17.25) (width 0.3) (layer "B.Cu") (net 20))
 (segment (start 49.605 24.87) (end 49.605 49.31) (width 0.3) (layer "B.Cu") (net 46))
 (segment (start 49.605 49.31) (end 48.335 50.58) (width 0.3) (layer "B.Cu") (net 46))
 (segment (start 49.605 10.18) (end 48.335 11.45) (width 0.3) (layer "B.Cu") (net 21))
 (segment (start 48.335 11.45) (end 48.335 35.89) (width 0.3) (layer "B.Cu") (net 21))
 (segment (start 48.335 43.51) (end 48.335 48.04) (width 0.3) (layer "B.Cu") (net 47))
 (segment (start 52.145 12.72) (end 52.145 35.89) (width 0.3) (layer "B.Cu") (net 22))
 (segment (start 52.145 43.51) (end 52.145 49.31) (width 0.3) (layer "B.Cu") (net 48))
 (segment (start 52.145 49.31) (end 50.875 50.58) (width 0.3) (layer "B.Cu") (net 48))
 (segment (start 52.145 10.18) (end 50.875 11.45) (width 0.3) (layer "B.Cu") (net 3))
 (segment (start 50.875 11.45) (end 50.875 30.38) (width 0.3) (layer "B.Cu") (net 3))
 (segment (start 50.875 30.38) (end 50.875 48.04) (width 0.3) (layer "B.Cu") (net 3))
 (segment (start 54.685 12.72) (end 54.685 26.57) (width 0.3) (layer "B.Cu") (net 23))
 (segment (start 54.685 34.19) (end 54.685 49.31) (width 0.3) (layer "B.Cu") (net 49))
 (segment (start 54.685 49.31) (end 53.415 50.58) (width 0.3) (layer "B.Cu") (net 49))
 (segment (start 54.685 10.18) (end 53.415 11.45) (width 0.3) (layer "B.Cu") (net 24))
 (segment (start 53.415 11.45) (end 53.415 17.25) (width 0.3) (layer "B.Cu") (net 24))
 (segment (start 53.415 24.87) (end 53.415 48.04) (width 0.3) (layer "B.Cu") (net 50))
 (segment (start 57.225 12.72) (end 57.225 17.25) (width 0.3) (layer "B.Cu") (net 25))
 (segment (start 57.225 24.87) (end 57.225 49.31) (width 0.3) (layer "B.Cu") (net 51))
 (segment (start 57.225 49.31) (end 55.955 50.58) (width 0.3) (layer "B.Cu") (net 51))
 (segment (start 57.225 10.18) (end 55.955 11.45) (width 0.3) (layer "B.Cu") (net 26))
 (segment (start 55.955 11.45) (end 55.955 35.89) (width 0.3) (layer "B.Cu") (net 26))
 (segment (start 55.955 43.51) (end 55.955 48.04) (width 0.3) (layer "B.Cu") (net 52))
 (segment (start 59.765 12.72) (end 59.765 30.38) (width 0.3) (layer "B.Cu") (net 3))
 (segment (start 59.765 30.38) (end 59.765 49.31) (width 0.3) (layer "B.Cu") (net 3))
 (segment (start 59.765 49.31) (end 58.495 50.58) (width 0.3) (layer "B.Cu") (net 3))
 (segment (start 59.765 10.18) (end 58.495 11.45) (width 0.3) (layer "B.Cu") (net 27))
 (segment (start 58.495 11.45) (end 58.495 26.57) (width 0.3) (layer "B.Cu") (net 27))
 (segment (start 58.495 34.19) (end 58.495 48.04) (width 0.3) (layer "B.Cu") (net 53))
 (gr_line (start 0 0) (end 70 0) (layer "Edge.Cuts") (width 0.1))
 (gr_line (start 70 0) (end 70 60.76) (layer "Edge.Cuts") (width 0.1))
 (gr_line (start 70 60.76) (end 0 60.76) (layer "Edge.Cuts") (width 0.1))
 (gr_line (start 0 60.76) (end 0 0) (layer "Edge.Cuts") (width 0.1)))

